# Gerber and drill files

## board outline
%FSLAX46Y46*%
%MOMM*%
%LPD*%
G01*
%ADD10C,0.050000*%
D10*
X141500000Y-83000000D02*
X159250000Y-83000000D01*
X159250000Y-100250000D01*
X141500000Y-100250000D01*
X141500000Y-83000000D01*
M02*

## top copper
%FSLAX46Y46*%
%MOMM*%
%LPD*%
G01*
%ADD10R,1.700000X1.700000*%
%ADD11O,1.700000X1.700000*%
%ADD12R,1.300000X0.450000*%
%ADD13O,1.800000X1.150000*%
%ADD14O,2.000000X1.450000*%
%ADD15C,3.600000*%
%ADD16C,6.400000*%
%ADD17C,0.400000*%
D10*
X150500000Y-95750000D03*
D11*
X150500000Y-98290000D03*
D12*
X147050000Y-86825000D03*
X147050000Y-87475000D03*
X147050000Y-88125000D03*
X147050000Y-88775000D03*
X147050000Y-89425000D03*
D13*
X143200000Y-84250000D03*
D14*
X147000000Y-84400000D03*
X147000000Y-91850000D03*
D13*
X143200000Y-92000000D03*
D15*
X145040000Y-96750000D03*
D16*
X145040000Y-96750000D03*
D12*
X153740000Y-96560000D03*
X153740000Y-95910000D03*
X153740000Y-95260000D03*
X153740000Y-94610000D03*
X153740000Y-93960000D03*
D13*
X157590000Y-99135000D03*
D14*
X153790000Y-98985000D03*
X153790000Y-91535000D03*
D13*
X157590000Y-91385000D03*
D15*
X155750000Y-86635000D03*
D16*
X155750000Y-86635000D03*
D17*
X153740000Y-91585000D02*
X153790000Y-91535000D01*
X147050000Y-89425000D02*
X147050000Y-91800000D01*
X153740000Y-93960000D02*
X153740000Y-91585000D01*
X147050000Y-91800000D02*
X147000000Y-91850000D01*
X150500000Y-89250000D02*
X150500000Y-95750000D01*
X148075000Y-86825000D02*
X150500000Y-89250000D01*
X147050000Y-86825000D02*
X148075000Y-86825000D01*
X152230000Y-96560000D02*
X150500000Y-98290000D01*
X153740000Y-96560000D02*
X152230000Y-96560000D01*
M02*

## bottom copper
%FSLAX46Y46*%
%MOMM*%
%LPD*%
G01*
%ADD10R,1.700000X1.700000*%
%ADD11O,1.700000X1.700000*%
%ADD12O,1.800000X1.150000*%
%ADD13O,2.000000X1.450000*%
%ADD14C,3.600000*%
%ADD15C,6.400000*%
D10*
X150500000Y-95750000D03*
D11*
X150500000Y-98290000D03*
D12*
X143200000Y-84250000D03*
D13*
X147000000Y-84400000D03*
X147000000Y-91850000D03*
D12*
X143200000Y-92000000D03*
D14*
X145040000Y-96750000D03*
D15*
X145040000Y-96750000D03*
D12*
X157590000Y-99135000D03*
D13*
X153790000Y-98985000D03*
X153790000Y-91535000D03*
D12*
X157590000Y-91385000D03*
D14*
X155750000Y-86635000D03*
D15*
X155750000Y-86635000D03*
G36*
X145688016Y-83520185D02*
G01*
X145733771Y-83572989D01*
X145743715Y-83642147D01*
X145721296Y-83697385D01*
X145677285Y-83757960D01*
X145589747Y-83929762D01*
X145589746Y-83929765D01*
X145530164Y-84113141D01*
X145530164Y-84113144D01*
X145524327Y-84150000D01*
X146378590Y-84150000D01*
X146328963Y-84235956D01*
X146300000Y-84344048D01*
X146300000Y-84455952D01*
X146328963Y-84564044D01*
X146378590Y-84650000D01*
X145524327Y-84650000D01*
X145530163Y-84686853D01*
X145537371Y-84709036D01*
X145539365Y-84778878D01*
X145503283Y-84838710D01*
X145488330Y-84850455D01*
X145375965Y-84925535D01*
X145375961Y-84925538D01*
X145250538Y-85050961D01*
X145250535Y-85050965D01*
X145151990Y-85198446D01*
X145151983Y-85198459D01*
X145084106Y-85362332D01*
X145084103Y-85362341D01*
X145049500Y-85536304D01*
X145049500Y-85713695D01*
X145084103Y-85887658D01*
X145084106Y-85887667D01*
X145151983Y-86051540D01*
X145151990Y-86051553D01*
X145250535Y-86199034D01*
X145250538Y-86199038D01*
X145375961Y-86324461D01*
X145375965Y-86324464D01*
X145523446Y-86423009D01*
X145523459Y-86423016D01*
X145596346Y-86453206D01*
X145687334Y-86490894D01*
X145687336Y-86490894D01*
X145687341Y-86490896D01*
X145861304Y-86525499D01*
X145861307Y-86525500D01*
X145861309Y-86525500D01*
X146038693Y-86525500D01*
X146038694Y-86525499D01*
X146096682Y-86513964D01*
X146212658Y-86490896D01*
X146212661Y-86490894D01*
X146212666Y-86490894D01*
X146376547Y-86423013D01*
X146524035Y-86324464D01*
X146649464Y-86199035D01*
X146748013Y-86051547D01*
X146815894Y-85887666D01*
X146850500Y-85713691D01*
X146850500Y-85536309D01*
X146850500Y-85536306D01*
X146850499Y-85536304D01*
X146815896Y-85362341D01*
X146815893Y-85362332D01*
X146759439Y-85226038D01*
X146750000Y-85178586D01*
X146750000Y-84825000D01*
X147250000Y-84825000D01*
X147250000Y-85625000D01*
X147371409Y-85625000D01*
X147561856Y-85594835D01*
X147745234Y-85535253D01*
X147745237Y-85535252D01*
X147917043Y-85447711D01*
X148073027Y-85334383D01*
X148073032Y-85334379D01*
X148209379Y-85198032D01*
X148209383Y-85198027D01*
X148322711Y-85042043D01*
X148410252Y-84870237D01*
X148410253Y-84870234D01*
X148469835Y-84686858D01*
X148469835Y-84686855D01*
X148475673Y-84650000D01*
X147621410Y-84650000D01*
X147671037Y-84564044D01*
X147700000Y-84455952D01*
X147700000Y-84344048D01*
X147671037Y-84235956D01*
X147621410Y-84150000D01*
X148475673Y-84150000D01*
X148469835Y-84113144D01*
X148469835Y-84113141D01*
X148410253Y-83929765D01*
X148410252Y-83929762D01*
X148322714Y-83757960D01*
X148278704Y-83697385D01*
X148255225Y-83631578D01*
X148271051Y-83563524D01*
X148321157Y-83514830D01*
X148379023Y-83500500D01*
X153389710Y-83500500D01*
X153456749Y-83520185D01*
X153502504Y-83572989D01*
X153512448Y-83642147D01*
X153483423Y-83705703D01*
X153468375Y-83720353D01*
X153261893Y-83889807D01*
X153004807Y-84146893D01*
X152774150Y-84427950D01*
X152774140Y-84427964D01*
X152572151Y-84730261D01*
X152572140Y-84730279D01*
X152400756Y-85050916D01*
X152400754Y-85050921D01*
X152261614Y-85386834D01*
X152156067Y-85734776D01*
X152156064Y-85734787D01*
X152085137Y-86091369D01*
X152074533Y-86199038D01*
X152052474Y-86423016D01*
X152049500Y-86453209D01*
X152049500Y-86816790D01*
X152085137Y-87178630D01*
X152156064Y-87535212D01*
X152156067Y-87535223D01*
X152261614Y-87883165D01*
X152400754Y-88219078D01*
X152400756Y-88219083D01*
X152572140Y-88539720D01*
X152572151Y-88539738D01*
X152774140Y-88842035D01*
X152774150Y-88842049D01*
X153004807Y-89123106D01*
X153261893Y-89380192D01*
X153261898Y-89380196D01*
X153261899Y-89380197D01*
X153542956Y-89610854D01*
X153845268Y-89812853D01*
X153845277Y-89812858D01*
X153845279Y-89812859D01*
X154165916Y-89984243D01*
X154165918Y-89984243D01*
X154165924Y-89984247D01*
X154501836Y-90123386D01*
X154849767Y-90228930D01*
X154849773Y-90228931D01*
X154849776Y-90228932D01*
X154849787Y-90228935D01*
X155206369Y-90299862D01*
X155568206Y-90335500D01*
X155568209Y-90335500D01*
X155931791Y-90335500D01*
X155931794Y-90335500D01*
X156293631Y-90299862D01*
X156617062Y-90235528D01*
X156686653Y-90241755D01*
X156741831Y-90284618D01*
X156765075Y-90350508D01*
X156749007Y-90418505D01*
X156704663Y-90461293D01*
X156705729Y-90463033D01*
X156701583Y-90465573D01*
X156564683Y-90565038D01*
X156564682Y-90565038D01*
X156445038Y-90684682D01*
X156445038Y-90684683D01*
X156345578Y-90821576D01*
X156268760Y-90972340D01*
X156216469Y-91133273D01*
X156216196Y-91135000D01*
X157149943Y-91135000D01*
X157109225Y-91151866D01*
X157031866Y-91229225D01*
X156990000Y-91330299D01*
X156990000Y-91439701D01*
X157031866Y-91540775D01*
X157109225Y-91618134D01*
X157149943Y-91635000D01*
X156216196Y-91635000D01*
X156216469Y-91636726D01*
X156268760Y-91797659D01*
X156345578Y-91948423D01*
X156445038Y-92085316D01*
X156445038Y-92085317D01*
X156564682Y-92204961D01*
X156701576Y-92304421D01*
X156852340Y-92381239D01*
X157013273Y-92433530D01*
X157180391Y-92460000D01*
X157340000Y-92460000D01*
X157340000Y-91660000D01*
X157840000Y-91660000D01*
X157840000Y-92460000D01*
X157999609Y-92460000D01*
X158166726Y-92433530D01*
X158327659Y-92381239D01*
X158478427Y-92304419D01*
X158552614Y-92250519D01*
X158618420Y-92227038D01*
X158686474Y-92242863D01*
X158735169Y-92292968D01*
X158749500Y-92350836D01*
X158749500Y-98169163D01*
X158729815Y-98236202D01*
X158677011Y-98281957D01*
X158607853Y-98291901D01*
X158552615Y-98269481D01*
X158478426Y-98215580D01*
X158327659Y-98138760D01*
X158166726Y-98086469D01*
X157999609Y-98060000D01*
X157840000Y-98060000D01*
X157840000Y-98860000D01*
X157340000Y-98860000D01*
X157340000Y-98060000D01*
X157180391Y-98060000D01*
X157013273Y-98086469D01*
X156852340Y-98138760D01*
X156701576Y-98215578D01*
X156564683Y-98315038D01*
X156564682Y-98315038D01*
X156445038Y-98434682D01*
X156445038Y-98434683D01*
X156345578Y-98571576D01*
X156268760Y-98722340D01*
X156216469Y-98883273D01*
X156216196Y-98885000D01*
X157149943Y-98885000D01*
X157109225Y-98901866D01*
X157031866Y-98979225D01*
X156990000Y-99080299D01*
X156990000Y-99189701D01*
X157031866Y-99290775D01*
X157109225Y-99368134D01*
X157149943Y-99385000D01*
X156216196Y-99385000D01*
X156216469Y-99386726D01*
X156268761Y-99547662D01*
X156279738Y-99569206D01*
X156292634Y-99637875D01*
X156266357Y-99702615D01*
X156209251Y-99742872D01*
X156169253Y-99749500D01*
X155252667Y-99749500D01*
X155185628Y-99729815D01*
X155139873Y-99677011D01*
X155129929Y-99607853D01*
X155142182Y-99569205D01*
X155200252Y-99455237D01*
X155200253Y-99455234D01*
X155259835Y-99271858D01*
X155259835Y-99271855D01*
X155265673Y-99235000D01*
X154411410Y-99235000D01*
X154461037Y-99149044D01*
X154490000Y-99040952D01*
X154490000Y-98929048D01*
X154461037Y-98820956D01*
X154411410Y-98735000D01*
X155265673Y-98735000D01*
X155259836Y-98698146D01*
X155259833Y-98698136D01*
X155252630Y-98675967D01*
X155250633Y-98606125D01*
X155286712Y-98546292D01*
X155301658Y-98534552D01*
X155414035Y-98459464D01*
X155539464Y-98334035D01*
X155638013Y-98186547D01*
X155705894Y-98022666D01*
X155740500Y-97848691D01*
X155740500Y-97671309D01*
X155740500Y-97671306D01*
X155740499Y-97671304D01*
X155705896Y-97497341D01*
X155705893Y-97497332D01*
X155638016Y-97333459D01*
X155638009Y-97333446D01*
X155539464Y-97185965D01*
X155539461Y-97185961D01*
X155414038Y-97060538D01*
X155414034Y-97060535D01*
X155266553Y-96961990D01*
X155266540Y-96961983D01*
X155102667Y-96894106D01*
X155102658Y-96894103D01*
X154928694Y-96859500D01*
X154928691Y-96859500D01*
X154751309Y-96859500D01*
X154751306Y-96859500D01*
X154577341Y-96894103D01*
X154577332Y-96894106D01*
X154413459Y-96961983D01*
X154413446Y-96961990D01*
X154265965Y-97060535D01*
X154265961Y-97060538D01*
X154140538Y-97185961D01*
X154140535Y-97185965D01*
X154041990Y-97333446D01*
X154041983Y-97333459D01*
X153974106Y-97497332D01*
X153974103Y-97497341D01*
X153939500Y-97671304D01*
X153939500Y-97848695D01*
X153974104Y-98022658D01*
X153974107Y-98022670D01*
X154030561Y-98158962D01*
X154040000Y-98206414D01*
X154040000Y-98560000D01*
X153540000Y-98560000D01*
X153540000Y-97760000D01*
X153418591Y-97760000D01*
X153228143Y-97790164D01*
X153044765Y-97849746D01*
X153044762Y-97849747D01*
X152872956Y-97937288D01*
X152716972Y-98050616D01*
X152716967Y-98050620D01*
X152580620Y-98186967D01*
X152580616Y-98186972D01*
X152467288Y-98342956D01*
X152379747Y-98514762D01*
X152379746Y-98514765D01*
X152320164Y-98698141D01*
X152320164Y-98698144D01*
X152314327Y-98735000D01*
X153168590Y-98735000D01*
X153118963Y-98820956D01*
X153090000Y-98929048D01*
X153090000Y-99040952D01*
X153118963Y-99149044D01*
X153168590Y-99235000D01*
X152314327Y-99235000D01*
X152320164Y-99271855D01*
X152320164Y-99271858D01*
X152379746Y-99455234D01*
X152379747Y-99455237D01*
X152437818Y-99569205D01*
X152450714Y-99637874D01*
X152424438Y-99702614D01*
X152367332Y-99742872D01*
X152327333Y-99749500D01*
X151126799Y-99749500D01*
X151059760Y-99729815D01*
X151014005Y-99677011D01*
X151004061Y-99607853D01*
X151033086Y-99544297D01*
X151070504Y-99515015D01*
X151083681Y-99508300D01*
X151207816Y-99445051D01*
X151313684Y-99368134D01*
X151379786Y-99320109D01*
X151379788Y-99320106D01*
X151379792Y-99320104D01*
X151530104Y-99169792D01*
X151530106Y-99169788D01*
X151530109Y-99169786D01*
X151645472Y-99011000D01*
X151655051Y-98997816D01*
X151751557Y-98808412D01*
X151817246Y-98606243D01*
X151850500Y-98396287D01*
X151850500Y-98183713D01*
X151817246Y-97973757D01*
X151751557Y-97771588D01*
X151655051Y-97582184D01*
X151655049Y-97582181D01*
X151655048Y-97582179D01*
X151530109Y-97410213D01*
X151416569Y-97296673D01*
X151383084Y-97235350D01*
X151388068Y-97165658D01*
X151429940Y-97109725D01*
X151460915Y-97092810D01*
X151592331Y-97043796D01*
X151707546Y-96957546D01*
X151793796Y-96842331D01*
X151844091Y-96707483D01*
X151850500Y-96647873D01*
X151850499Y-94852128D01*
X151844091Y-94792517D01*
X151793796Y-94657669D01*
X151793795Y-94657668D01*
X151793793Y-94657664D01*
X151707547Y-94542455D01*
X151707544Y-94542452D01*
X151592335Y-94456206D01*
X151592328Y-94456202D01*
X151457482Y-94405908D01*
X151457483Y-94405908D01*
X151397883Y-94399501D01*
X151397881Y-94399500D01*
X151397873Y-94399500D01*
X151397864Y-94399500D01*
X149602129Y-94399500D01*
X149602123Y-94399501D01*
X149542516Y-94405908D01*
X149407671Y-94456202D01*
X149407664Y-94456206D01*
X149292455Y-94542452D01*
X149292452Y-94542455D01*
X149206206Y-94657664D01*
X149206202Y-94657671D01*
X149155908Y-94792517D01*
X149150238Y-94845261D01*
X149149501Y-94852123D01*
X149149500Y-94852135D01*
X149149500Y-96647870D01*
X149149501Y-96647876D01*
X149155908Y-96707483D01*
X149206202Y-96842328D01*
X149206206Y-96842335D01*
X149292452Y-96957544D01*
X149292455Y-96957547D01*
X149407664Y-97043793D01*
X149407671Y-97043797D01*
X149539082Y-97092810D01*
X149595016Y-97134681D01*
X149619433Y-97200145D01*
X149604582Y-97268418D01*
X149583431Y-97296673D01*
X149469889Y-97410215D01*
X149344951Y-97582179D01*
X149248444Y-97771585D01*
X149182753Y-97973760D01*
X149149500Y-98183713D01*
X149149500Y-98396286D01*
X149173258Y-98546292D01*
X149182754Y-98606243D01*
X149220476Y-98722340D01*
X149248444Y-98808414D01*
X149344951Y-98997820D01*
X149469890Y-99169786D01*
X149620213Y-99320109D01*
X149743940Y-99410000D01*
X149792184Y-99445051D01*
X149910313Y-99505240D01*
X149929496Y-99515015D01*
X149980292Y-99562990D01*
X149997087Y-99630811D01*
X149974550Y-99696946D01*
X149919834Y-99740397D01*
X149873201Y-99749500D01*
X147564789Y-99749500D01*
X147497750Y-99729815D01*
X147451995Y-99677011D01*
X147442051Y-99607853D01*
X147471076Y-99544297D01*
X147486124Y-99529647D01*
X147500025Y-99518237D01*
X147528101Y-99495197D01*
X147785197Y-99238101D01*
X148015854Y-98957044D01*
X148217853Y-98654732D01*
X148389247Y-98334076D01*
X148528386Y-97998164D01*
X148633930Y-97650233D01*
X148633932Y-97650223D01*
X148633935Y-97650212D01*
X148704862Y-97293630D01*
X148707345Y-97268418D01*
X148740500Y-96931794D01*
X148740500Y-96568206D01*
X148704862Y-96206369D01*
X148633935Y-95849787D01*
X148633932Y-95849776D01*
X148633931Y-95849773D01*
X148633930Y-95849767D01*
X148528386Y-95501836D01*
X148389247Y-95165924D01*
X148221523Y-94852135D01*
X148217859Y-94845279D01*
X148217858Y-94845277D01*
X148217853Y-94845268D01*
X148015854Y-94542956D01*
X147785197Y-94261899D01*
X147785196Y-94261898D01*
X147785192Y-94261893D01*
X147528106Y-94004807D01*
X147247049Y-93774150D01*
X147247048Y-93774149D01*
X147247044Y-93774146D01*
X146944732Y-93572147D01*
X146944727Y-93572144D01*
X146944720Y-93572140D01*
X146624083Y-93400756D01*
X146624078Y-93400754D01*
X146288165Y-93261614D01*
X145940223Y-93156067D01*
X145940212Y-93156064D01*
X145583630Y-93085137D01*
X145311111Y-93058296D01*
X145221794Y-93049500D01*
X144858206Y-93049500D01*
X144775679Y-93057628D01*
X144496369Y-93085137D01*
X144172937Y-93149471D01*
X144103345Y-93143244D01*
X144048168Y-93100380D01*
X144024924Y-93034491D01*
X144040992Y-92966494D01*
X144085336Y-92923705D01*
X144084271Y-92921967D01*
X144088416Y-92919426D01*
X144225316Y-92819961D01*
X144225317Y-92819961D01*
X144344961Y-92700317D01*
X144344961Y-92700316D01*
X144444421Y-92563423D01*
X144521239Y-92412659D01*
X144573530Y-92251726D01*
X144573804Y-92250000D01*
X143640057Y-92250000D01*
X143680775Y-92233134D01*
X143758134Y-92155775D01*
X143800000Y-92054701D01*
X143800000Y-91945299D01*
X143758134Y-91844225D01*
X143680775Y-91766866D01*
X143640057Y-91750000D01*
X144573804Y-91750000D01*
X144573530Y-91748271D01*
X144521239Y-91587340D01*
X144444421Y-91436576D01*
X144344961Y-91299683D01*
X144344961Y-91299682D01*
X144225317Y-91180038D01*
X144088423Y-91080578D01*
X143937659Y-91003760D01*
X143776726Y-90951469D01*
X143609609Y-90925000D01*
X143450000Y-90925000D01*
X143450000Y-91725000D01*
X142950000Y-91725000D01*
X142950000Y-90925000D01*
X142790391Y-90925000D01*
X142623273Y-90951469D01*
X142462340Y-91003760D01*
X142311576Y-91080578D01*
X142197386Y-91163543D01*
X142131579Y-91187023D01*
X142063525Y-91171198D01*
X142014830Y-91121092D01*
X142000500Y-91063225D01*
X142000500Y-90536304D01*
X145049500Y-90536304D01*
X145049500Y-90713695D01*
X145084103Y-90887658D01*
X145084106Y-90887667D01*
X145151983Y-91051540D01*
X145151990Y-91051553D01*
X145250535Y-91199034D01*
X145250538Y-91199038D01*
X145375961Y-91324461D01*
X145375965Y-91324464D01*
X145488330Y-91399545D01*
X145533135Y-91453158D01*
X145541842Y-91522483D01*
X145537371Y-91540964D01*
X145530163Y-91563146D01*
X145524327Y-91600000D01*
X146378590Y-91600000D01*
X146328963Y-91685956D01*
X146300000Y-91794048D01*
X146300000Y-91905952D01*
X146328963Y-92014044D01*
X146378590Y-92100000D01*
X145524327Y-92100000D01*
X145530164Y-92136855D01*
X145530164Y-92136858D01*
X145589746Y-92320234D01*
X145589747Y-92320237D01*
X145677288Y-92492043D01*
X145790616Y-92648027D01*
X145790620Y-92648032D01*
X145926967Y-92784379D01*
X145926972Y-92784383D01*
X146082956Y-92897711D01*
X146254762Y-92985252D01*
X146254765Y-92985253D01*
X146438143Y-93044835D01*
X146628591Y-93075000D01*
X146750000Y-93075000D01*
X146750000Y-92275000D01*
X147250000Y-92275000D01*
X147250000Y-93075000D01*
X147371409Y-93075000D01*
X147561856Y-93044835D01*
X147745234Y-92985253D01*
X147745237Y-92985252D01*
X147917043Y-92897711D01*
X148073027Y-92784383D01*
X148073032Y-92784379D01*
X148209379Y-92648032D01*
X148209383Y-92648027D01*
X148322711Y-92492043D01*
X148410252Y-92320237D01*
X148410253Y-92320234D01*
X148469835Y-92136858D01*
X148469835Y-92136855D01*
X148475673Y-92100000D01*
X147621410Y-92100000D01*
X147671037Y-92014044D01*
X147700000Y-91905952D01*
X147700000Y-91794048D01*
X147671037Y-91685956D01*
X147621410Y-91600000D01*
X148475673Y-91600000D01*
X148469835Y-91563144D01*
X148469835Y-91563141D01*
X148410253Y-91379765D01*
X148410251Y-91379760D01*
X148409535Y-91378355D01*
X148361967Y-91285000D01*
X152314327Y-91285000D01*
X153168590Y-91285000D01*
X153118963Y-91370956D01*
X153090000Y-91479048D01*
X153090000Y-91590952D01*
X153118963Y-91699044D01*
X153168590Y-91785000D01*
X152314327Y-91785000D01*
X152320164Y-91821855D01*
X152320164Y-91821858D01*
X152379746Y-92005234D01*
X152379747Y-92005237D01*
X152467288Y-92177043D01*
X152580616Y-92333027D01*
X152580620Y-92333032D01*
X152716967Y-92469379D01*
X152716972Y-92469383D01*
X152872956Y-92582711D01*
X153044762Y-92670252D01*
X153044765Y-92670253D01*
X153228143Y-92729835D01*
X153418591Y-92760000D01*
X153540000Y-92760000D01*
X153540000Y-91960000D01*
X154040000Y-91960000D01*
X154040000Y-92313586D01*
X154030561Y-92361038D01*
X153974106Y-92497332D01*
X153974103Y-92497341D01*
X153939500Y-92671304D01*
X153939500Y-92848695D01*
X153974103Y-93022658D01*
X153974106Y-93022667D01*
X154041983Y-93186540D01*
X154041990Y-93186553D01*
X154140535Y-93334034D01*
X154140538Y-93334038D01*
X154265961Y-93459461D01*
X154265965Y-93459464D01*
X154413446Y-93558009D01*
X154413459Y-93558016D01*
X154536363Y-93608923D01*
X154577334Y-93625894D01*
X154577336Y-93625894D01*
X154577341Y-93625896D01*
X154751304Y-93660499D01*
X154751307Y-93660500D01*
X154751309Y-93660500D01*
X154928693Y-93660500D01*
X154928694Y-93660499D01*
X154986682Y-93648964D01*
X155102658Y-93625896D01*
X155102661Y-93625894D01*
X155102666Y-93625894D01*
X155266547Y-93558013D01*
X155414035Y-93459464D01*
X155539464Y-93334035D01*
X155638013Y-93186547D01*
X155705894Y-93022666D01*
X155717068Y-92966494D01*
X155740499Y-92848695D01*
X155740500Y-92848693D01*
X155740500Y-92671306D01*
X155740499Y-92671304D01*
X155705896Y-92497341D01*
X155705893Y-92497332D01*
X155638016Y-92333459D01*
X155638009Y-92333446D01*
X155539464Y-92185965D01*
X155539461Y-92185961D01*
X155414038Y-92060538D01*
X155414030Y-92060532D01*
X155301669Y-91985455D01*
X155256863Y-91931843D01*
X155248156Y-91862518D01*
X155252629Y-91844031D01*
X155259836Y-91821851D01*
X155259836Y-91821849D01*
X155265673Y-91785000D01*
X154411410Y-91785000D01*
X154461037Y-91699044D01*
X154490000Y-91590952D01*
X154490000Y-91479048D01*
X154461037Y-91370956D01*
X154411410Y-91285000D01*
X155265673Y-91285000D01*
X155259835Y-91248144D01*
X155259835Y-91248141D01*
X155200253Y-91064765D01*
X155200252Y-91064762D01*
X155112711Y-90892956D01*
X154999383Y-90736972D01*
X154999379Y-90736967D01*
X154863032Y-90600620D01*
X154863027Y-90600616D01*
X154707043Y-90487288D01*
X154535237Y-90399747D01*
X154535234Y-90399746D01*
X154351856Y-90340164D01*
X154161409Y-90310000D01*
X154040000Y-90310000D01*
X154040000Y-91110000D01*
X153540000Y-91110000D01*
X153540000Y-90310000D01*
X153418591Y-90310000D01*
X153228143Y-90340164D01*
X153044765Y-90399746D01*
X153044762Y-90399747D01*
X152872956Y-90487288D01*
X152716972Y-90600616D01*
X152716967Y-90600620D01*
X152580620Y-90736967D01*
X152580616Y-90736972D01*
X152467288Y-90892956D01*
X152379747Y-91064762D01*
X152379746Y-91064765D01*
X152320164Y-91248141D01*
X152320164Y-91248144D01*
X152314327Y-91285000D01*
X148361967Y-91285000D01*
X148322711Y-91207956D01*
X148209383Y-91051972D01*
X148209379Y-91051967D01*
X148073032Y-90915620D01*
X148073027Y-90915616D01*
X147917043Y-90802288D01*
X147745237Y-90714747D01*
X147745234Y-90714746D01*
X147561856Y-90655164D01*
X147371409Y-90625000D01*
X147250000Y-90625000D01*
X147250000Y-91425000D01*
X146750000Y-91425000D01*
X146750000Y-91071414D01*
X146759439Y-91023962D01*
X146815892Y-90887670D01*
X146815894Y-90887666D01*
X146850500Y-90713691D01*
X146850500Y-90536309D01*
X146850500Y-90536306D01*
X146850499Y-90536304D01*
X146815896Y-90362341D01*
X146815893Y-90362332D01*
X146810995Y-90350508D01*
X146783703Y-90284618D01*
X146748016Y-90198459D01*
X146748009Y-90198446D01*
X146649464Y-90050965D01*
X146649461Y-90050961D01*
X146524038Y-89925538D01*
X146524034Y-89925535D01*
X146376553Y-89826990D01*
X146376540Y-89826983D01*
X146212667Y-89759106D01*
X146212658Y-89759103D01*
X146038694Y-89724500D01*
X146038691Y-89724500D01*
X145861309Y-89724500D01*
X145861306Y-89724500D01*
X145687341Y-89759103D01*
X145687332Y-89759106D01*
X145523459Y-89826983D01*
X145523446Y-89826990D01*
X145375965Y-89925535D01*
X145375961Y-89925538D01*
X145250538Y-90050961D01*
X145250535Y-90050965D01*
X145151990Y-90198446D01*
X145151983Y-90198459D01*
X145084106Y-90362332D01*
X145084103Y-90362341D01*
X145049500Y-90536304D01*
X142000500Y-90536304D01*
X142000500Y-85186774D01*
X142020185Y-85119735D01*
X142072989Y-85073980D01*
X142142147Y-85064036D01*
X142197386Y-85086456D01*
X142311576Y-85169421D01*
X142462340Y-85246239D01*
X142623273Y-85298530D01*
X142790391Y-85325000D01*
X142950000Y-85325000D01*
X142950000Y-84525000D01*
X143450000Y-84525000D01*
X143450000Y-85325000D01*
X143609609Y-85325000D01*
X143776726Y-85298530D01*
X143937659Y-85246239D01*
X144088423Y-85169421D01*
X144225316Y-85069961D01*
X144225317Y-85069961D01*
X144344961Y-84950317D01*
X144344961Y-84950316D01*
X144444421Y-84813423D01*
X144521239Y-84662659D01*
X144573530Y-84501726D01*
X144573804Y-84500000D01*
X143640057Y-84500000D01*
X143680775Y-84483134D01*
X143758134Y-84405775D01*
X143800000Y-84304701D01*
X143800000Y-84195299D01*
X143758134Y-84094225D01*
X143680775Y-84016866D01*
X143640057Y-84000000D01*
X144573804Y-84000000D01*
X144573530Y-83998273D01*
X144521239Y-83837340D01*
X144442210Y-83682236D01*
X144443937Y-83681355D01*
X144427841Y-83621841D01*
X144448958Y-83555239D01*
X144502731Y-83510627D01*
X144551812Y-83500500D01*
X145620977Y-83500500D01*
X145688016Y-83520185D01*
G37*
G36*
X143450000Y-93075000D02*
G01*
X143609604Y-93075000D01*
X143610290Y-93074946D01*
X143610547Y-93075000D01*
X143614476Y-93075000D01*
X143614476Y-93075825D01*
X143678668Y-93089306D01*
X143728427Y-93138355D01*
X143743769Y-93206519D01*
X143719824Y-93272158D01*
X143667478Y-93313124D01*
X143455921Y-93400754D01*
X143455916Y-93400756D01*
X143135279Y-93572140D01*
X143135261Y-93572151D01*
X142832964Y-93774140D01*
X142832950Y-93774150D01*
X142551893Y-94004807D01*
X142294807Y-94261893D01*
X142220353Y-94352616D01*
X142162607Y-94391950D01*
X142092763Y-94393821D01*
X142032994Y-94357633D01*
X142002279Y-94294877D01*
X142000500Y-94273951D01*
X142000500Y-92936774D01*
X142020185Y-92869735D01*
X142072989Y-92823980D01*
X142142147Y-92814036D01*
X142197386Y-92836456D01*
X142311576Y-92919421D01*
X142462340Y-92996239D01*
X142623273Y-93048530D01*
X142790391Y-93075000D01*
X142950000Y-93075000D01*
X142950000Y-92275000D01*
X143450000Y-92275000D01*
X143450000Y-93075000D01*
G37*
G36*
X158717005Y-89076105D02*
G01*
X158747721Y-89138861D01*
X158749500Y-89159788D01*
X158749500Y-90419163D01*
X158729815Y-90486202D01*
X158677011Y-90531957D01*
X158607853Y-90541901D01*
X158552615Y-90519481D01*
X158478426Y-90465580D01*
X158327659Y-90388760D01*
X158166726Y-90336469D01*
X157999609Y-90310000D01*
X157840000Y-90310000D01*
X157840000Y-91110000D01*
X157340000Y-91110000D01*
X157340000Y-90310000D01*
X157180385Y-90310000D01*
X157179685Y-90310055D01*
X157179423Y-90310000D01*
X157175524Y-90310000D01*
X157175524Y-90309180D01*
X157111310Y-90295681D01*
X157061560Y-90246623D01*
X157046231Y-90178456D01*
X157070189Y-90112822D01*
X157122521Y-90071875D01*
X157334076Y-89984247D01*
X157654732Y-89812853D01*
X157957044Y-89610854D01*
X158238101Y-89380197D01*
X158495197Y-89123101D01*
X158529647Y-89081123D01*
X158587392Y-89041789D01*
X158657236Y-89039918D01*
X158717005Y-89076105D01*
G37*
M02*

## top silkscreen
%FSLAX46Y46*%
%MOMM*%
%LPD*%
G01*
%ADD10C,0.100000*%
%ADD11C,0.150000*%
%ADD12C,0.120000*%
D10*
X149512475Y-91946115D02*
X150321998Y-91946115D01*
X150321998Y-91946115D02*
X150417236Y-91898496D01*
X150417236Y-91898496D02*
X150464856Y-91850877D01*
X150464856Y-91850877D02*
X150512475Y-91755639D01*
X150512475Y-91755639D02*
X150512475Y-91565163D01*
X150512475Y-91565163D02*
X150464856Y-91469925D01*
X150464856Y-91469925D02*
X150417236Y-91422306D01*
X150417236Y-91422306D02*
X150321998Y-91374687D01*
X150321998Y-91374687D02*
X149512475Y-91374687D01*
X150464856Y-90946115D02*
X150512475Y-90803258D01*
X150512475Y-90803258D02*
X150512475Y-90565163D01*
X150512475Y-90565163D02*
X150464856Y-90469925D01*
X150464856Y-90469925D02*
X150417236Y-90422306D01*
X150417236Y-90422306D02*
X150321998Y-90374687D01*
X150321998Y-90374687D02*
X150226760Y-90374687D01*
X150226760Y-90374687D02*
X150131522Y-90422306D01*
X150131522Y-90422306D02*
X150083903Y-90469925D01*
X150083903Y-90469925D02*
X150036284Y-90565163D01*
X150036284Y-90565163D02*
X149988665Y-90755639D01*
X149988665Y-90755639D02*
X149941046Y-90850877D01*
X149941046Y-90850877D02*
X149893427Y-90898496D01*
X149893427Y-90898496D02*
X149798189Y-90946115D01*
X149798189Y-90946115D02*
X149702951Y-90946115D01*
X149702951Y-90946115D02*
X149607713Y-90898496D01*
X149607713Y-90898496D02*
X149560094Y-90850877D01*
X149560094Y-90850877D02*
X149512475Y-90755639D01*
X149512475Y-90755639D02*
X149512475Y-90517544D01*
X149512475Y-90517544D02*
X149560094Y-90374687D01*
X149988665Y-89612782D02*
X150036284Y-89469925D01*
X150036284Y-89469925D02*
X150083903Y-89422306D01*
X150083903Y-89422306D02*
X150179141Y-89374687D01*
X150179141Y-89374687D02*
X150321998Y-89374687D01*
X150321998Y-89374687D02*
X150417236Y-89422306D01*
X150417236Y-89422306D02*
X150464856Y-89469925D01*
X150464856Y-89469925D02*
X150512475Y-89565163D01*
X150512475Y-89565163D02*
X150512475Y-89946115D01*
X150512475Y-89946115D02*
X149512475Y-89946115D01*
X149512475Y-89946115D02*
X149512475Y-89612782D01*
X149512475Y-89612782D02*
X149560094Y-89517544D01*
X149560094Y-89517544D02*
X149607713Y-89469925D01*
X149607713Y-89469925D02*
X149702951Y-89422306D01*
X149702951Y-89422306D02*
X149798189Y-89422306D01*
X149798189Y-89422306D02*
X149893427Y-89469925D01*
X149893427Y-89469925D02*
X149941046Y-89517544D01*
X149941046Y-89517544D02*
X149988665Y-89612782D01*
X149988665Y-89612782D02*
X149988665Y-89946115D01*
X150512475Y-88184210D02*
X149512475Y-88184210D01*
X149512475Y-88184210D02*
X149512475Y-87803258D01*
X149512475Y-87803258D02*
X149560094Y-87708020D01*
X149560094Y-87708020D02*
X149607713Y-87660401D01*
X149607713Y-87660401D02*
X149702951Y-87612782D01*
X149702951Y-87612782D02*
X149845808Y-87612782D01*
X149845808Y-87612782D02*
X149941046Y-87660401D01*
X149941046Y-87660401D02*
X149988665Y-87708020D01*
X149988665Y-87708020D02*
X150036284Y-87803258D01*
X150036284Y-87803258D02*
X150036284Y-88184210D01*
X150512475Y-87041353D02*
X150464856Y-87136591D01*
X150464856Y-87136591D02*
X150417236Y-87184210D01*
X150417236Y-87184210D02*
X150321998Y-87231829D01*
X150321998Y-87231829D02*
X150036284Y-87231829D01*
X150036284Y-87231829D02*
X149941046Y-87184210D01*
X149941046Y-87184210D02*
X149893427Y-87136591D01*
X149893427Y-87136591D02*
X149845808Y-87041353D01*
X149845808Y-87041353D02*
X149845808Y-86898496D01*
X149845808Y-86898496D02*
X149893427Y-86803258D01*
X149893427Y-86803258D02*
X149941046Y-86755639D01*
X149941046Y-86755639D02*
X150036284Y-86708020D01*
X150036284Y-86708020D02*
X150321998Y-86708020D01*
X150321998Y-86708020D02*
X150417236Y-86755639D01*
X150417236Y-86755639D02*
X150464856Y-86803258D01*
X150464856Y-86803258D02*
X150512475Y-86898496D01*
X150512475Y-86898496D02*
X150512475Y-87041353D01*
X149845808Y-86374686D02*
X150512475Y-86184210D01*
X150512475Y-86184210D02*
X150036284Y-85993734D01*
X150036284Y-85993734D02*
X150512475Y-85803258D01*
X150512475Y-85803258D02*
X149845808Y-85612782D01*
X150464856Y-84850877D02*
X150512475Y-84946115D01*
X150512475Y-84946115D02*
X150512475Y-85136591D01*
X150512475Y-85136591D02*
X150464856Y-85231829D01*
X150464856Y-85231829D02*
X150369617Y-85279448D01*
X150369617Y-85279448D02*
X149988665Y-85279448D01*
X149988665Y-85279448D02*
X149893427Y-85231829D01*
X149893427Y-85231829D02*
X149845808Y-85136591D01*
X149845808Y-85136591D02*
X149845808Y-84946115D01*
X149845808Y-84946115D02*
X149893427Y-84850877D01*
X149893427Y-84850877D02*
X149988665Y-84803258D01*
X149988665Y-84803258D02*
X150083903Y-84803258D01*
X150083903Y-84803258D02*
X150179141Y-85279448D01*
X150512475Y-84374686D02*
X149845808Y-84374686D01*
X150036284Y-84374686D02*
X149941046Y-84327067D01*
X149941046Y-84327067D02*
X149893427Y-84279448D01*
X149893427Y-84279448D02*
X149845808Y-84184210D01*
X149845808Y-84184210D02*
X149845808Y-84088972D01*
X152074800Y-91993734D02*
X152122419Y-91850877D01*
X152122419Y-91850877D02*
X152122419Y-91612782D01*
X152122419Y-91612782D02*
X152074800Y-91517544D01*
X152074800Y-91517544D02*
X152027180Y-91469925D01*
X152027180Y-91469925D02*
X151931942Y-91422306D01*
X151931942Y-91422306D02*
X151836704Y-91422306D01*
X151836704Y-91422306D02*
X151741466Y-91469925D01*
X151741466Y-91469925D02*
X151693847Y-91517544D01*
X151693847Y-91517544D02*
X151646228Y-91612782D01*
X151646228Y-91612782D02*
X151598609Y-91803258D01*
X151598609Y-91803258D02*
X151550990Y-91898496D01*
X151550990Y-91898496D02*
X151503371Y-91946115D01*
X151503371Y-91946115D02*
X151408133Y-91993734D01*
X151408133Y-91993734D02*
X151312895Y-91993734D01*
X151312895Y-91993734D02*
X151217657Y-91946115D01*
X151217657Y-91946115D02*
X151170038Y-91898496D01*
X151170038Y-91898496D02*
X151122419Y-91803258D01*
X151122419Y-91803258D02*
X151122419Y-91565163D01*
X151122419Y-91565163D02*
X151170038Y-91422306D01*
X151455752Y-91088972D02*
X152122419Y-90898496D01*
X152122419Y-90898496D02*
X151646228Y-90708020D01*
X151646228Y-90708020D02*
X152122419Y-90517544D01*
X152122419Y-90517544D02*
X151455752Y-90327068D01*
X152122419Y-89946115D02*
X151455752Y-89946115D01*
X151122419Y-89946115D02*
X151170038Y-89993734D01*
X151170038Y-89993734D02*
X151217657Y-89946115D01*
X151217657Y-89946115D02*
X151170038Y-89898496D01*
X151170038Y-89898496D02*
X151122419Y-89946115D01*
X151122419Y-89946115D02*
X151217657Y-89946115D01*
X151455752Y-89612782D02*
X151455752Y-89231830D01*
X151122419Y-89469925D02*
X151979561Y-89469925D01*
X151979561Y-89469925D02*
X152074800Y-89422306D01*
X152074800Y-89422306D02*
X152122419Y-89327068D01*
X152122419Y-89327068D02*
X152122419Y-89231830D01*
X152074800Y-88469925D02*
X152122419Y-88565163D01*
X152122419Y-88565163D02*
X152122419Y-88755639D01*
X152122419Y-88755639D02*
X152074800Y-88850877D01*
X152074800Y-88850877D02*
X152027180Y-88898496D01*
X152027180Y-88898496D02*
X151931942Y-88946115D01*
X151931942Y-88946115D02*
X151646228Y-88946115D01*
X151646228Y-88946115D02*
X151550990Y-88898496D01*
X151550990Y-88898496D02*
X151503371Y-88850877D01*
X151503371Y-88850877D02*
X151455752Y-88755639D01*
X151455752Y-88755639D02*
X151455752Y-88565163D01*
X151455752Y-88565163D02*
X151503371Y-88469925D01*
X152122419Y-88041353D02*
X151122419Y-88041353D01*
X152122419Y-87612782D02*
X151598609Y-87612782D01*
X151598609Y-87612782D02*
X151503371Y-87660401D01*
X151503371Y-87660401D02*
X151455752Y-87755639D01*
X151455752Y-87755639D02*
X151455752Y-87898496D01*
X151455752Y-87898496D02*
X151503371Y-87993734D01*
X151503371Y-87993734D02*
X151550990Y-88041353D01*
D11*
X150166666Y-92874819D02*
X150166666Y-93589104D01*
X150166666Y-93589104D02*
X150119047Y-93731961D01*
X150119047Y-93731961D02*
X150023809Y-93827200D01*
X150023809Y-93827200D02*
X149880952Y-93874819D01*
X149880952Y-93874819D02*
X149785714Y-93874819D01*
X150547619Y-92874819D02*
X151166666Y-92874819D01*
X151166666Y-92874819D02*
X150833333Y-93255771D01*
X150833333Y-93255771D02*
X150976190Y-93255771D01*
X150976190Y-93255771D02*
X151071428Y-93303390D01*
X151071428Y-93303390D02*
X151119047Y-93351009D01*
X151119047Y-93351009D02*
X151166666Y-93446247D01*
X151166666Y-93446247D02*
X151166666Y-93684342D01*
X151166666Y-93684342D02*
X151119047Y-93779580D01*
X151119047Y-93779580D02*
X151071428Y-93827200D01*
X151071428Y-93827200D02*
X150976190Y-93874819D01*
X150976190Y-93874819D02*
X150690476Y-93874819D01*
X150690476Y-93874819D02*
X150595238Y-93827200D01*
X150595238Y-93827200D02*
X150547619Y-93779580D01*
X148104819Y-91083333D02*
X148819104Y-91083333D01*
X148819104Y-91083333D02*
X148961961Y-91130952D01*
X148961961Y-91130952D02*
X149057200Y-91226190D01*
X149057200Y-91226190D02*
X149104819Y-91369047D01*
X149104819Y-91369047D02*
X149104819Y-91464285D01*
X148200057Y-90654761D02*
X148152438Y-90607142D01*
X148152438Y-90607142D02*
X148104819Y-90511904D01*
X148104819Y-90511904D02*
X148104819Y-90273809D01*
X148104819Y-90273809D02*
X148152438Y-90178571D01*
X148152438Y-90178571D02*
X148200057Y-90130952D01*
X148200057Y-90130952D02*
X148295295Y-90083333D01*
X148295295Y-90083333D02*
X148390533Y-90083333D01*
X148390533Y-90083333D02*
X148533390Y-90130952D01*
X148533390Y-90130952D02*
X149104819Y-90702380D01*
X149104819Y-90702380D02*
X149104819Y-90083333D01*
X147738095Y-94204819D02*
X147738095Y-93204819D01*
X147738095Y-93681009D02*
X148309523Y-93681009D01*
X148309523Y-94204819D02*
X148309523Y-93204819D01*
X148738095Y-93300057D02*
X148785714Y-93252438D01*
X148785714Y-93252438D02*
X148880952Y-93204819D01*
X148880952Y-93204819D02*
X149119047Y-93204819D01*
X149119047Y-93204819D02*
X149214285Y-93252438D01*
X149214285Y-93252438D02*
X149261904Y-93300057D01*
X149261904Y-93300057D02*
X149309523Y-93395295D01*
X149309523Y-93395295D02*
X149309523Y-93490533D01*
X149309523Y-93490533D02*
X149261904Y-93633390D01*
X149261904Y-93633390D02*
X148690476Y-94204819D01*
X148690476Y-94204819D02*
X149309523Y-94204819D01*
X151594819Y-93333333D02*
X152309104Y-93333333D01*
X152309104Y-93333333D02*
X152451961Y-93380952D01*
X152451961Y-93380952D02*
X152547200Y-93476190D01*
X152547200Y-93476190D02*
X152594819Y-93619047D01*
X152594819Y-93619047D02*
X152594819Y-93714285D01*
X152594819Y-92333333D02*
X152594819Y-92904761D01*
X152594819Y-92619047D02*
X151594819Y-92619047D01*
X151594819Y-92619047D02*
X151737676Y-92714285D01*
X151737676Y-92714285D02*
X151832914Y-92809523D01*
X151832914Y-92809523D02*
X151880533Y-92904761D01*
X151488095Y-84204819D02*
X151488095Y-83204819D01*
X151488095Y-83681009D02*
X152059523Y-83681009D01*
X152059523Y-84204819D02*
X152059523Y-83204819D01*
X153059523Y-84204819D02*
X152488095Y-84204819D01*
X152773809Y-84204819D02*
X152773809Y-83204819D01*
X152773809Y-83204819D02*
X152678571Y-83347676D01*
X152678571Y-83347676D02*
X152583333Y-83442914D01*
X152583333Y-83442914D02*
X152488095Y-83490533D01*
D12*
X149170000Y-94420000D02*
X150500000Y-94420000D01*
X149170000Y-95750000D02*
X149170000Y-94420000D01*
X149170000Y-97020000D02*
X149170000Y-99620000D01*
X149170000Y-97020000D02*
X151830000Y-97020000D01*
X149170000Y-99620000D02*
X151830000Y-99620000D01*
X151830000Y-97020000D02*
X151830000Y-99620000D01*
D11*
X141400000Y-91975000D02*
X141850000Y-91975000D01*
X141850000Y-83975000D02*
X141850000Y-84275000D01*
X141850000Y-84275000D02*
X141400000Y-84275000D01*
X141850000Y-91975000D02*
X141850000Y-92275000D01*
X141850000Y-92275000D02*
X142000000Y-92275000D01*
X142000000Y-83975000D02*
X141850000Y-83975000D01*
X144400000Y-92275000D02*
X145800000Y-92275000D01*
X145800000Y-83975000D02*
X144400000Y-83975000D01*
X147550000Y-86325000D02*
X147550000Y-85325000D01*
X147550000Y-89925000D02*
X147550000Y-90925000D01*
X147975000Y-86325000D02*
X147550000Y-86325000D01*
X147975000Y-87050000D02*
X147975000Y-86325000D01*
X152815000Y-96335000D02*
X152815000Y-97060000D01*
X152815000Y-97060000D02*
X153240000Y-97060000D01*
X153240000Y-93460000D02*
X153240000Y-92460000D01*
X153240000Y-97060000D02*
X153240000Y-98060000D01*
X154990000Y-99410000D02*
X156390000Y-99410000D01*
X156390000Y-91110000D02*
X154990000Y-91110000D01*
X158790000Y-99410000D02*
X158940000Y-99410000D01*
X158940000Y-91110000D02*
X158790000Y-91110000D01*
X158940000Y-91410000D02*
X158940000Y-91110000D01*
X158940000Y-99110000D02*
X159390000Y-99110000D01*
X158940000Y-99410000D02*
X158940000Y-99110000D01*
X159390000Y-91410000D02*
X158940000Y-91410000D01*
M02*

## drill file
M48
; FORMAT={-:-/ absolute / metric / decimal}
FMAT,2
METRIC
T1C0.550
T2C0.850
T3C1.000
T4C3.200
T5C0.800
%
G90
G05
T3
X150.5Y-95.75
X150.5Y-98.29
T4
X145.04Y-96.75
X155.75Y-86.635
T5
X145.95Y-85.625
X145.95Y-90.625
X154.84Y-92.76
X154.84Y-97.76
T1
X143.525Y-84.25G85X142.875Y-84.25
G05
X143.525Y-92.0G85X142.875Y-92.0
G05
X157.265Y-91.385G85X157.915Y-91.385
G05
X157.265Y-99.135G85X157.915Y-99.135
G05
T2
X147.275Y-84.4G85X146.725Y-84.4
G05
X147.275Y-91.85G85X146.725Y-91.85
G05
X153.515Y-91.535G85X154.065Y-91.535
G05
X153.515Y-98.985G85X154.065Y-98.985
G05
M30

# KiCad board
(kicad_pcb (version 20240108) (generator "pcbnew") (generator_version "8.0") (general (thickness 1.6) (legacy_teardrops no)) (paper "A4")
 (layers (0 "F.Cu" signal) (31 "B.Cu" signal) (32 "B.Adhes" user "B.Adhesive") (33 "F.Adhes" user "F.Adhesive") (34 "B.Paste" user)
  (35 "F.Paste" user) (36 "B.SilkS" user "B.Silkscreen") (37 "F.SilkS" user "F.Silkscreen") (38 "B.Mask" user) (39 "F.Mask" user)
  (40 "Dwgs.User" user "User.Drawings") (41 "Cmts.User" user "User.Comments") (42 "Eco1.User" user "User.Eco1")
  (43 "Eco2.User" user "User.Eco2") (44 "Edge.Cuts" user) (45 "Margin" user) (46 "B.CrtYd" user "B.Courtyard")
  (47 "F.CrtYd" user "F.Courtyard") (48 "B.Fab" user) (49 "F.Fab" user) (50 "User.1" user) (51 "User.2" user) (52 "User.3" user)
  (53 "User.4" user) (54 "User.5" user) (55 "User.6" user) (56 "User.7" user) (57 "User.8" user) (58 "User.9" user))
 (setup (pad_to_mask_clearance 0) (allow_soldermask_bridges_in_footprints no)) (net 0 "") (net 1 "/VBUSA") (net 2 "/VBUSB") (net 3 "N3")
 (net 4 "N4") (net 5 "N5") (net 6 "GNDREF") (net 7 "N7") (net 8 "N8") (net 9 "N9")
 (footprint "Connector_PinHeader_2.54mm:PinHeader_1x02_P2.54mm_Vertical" (layer "F.Cu") (at 150.5 95.75)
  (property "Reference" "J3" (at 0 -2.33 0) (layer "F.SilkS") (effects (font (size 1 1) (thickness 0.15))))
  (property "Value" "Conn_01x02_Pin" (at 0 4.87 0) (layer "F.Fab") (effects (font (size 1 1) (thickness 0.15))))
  (fp_line (start -1.33 -1.33) (end 0 -1.33) (stroke (width 0.12) (type solid)) (layer "F.SilkS"))
  (fp_line (start -1.33 0) (end -1.33 -1.33) (stroke (width 0.12) (type solid)) (layer "F.SilkS"))
  (fp_line (start -1.33 1.27) (end -1.33 3.87) (stroke (width 0.12) (type solid)) (layer "F.SilkS"))
  (fp_line (start -1.33 1.27) (end 1.33 1.27) (stroke (width 0.12) (type solid)) (layer "F.SilkS"))
  (fp_line (start -1.33 3.87) (end 1.33 3.87) (stroke (width 0.12) (type solid)) (layer "F.SilkS"))
  (fp_line (start 1.33 1.27) (end 1.33 3.87) (stroke (width 0.12) (type solid)) (layer "F.SilkS"))
  (pad "1" thru_hole rect (at 0 0) (size 1.7 1.7) (drill 1) (layers "*.Cu" "*.Mask") (remove_unused_layers no) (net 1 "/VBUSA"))
  (pad "2" thru_hole oval (at 0 2.54) (size 1.7 1.7) (drill 1) (layers "*.Cu" "*.Mask") (remove_unused_layers no) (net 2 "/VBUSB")))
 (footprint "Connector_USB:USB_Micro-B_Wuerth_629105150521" (layer "F.Cu") (at 145.15 88.125 -90)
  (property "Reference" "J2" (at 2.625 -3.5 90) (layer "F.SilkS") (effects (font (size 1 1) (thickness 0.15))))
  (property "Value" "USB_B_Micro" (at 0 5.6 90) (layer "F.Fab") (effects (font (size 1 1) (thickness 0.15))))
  (fp_line (start 3.85 3.75) (end 3.85 3.3) (stroke (width 0.15) (type solid)) (layer "F.SilkS"))
  (fp_line (start -4.15 3.3) (end -3.85 3.3) (stroke (width 0.15) (type solid)) (layer "F.SilkS"))
  (fp_line (start -3.85 3.3) (end -3.85 3.75) (stroke (width 0.15) (type solid)) (layer "F.SilkS"))
  (fp_line (start 3.85 3.3) (end 4.15 3.3) (stroke (width 0.15) (type solid)) (layer "F.SilkS"))
  (fp_line (start 4.15 3.3) (end 4.15 3.15) (stroke (width 0.15) (type solid)) (layer "F.SilkS"))
  (fp_line (start -4.15 3.15) (end -4.15 3.3) (stroke (width 0.15) (type solid)) (layer "F.SilkS"))
  (fp_line (start 4.15 0.75) (end 4.15 -0.65) (stroke (width 0.15) (type solid)) (layer "F.SilkS"))
  (fp_line (start -4.15 -0.65) (end -4.15 0.75) (stroke (width 0.15) (type solid)) (layer "F.SilkS"))
  (fp_line (start -1.8 -2.4) (end -2.8 -2.4) (stroke (width 0.15) (type solid)) (layer "F.SilkS"))
  (fp_line (start 1.8 -2.4) (end 2.8 -2.4) (stroke (width 0.15) (type solid)) (layer "F.SilkS"))
  (fp_line (start -1.8 -2.825) (end -1.8 -2.4) (stroke (width 0.15) (type solid)) (layer "F.SilkS"))
  (fp_line (start -1.075 -2.825) (end -1.8 -2.825) (stroke (width 0.15) (type solid)) (layer "F.SilkS"))
  (pad "" np_thru_hole oval (at -2.5 -0.8 270) (size 0.8 0.8) (drill 0.8) (layers "*.Cu" "*.Mask"))
  (pad "" np_thru_hole oval (at 2.5 -0.8 270) (size 0.8 0.8) (drill 0.8) (layers "*.Cu" "*.Mask"))
  (pad "1" smd rect (at -1.3 -1.9 270) (size 0.45 1.3) (layers "F.Cu" "F.Paste" "F.Mask") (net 1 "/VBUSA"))
  (pad "2" smd rect (at -0.65 -1.9 270) (size 0.45 1.3) (layers "F.Cu" "F.Paste" "F.Mask") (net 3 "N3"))
  (pad "3" smd rect (at 0 -1.9 270) (size 0.45 1.3) (layers "F.Cu" "F.Paste" "F.Mask") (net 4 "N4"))
  (pad "4" smd rect (at 0.65 -1.9 270) (size 0.45 1.3) (layers "F.Cu" "F.Paste" "F.Mask") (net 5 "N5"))
  (pad "5" smd rect (at 1.3 -1.9 270) (size 0.45 1.3) (layers "F.Cu" "F.Paste" "F.Mask") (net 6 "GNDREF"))
  (pad "6" thru_hole oval (at -3.875 1.95 270) (size 1.15 1.8) (drill oval 0.55 1.2) (layers "*.Cu" "*.Mask") (remove_unused_layers no)
   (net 6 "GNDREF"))
  (pad "6" thru_hole oval (at -3.725 -1.85 270) (size 1.45 2) (drill oval 0.85 1.4) (layers "*.Cu" "*.Mask") (remove_unused_layers no)
   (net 6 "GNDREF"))
  (pad "6" thru_hole oval (at 3.725 -1.85 270) (size 1.45 2) (drill oval 0.85 1.4) (layers "*.Cu" "*.Mask") (remove_unused_layers no)
   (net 6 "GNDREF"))
  (pad "6" thru_hole oval (at 3.875 1.95 270) (size 1.15 1.8) (drill oval 0.55 1.2) (layers "*.Cu" "*.Mask") (remove_unused_layers no)
   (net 6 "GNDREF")))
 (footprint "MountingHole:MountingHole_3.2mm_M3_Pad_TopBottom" (layer "F.Cu") (at 145.04 96.75)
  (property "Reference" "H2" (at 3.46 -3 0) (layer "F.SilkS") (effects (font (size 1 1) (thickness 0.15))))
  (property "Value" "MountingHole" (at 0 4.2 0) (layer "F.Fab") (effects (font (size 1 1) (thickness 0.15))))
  (pad "1" thru_hole circle (at 0 0) (size 3.6 3.6) (drill 3.2) (layers "*.Cu" "*.Mask") (remove_unused_layers no))
  (pad "1" connect circle (at 0 0) (size 6.4 6.4) (layers "F.Cu" "F.Mask"))
  (pad "1" connect circle (at 0 0) (size 6.4 6.4) (layers "B.Cu" "B.Mask")))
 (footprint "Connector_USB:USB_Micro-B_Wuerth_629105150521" (layer "F.Cu") (at 155.64 95.26 90)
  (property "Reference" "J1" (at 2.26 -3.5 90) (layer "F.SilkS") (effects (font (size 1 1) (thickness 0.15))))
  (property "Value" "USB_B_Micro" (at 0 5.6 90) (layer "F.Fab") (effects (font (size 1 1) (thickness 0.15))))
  (fp_line (start -1.075 -2.825) (end -1.8 -2.825) (stroke (width 0.15) (type solid)) (layer "F.SilkS"))
  (fp_line (start -1.8 -2.825) (end -1.8 -2.4) (stroke (width 0.15) (type solid)) (layer "F.SilkS"))
  (fp_line (start 1.8 -2.4) (end 2.8 -2.4) (stroke (width 0.15) (type solid)) (layer "F.SilkS"))
  (fp_line (start -1.8 -2.4) (end -2.8 -2.4) (stroke (width 0.15) (type solid)) (layer "F.SilkS"))
  (fp_line (start -4.15 -0.65) (end -4.15 0.75) (stroke (width 0.15) (type solid)) (layer "F.SilkS"))
  (fp_line (start 4.15 0.75) (end 4.15 -0.65) (stroke (width 0.15) (type solid)) (layer "F.SilkS"))
  (fp_line (start -4.15 3.15) (end -4.15 3.3) (stroke (width 0.15) (type solid)) (layer "F.SilkS"))
  (fp_line (start 4.15 3.3) (end 4.15 3.15) (stroke (width 0.15) (type solid)) (layer "F.SilkS"))
  (fp_line (start 3.85 3.3) (end 4.15 3.3) (stroke (width 0.15) (type solid)) (layer "F.SilkS"))
  (fp_line (start -3.85 3.3) (end -3.85 3.75) (stroke (width 0.15) (type solid)) (layer "F.SilkS"))
  (fp_line (start -4.15 3.3) (end -3.85 3.3) (stroke (width 0.15) (type solid)) (layer "F.SilkS"))
  (fp_line (start 3.85 3.75) (end 3.85 3.3) (stroke (width 0.15) (type solid)) (layer "F.SilkS"))
  (pad "" np_thru_hole oval (at -2.5 -0.8 90) (size 0.8 0.8) (drill 0.8) (layers "*.Cu" "*.Mask"))
  (pad "" np_thru_hole oval (at 2.5 -0.8 90) (size 0.8 0.8) (drill 0.8) (layers "*.Cu" "*.Mask"))
  (pad "1" smd rect (at -1.3 -1.9 90) (size 0.45 1.3) (layers "F.Cu" "F.Paste" "F.Mask") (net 2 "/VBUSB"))
  (pad "2" smd rect (at -0.65 -1.9 90) (size 0.45 1.3) (layers "F.Cu" "F.Paste" "F.Mask") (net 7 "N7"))
  (pad "3" smd rect (at 0 -1.9 90) (size 0.45 1.3) (layers "F.Cu" "F.Paste" "F.Mask") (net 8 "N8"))
  (pad "4" smd rect (at 0.65 -1.9 90) (size 0.45 1.3) (layers "F.Cu" "F.Paste" "F.Mask") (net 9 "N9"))
  (pad "5" smd rect (at 1.3 -1.9 90) (size 0.45 1.3) (layers "F.Cu" "F.Paste" "F.Mask") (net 6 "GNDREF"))
  (pad "6" thru_hole oval (at -3.875 1.95 90) (size 1.15 1.8) (drill oval 0.55 1.2) (layers "*.Cu" "*.Mask") (remove_unused_layers no)
   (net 6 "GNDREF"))
  (pad "6" thru_hole oval (at -3.725 -1.85 90) (size 1.45 2) (drill oval 0.85 1.4) (layers "*.Cu" "*.Mask") (remove_unused_layers no)
   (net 6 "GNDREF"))
  (pad "6" thru_hole oval (at 3.725 -1.85 90) (size 1.45 2) (drill oval 0.85 1.4) (layers "*.Cu" "*.Mask") (remove_unused_layers no)
   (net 6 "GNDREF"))
  (pad "6" thru_hole oval (at 3.875 1.95 90) (size 1.15 1.8) (drill oval 0.55 1.2) (layers "*.Cu" "*.Mask") (remove_unused_layers no)
   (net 6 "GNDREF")))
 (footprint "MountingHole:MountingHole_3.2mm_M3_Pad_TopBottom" (layer "F.Cu") (at 155.75 86.635)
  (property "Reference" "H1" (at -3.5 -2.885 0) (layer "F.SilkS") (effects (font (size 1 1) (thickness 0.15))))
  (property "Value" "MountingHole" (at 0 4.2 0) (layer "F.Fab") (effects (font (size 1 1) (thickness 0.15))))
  (pad "1" thru_hole circle (at 0 0) (size 3.6 3.6) (drill 3.2) (layers "*.Cu" "*.Mask") (remove_unused_layers no))
  (pad "1" connect circle (at 0 0) (size 6.4 6.4) (layers "F.Cu" "F.Mask"))
  (pad "1" connect circle (at 0 0) (size 6.4 6.4) (layers "B.Cu" "B.Mask")))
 (gr_rect (start 141.5 83) (end 159.25 100.25) (stroke (width 0.05) (type default)) (fill none) (layer "Edge.Cuts"))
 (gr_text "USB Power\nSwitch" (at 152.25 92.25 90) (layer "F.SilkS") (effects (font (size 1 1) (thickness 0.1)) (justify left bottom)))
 (segment (start 153.74 91.585) (end 153.79 91.535) (width 0.4) (layer "F.Cu") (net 6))
 (segment (start 147.05 89.425) (end 147.05 91.8) (width 0.4) (layer "F.Cu") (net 6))
 (segment (start 153.74 93.96) (end 153.74 91.585) (width 0.4) (layer "F.Cu") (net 6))
 (segment (start 147.05 91.8) (end 147 91.85) (width 0.4) (layer "F.Cu") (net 6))
 (segment (start 150.5 89.25) (end 150.5 95.75) (width 0.4) (layer "F.Cu") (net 1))
 (segment (start 148.075 86.825) (end 150.5 89.25) (width 0.4) (layer "F.Cu") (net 1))
 (segment (start 147.05 86.825) (end 148.075 86.825) (width 0.4) (layer "F.Cu") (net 1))
 (segment (start 152.23 96.56) (end 150.5 98.29) (width 0.4) (layer "F.Cu") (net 2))
 (segment (start 153.74 96.56) (end 152.23 96.56) (width 0.4) (layer "F.Cu") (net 2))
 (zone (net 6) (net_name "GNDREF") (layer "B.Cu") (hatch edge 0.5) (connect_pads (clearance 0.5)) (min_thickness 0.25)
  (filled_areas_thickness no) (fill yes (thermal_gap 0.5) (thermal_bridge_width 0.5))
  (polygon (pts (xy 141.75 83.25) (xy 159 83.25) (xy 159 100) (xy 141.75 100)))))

